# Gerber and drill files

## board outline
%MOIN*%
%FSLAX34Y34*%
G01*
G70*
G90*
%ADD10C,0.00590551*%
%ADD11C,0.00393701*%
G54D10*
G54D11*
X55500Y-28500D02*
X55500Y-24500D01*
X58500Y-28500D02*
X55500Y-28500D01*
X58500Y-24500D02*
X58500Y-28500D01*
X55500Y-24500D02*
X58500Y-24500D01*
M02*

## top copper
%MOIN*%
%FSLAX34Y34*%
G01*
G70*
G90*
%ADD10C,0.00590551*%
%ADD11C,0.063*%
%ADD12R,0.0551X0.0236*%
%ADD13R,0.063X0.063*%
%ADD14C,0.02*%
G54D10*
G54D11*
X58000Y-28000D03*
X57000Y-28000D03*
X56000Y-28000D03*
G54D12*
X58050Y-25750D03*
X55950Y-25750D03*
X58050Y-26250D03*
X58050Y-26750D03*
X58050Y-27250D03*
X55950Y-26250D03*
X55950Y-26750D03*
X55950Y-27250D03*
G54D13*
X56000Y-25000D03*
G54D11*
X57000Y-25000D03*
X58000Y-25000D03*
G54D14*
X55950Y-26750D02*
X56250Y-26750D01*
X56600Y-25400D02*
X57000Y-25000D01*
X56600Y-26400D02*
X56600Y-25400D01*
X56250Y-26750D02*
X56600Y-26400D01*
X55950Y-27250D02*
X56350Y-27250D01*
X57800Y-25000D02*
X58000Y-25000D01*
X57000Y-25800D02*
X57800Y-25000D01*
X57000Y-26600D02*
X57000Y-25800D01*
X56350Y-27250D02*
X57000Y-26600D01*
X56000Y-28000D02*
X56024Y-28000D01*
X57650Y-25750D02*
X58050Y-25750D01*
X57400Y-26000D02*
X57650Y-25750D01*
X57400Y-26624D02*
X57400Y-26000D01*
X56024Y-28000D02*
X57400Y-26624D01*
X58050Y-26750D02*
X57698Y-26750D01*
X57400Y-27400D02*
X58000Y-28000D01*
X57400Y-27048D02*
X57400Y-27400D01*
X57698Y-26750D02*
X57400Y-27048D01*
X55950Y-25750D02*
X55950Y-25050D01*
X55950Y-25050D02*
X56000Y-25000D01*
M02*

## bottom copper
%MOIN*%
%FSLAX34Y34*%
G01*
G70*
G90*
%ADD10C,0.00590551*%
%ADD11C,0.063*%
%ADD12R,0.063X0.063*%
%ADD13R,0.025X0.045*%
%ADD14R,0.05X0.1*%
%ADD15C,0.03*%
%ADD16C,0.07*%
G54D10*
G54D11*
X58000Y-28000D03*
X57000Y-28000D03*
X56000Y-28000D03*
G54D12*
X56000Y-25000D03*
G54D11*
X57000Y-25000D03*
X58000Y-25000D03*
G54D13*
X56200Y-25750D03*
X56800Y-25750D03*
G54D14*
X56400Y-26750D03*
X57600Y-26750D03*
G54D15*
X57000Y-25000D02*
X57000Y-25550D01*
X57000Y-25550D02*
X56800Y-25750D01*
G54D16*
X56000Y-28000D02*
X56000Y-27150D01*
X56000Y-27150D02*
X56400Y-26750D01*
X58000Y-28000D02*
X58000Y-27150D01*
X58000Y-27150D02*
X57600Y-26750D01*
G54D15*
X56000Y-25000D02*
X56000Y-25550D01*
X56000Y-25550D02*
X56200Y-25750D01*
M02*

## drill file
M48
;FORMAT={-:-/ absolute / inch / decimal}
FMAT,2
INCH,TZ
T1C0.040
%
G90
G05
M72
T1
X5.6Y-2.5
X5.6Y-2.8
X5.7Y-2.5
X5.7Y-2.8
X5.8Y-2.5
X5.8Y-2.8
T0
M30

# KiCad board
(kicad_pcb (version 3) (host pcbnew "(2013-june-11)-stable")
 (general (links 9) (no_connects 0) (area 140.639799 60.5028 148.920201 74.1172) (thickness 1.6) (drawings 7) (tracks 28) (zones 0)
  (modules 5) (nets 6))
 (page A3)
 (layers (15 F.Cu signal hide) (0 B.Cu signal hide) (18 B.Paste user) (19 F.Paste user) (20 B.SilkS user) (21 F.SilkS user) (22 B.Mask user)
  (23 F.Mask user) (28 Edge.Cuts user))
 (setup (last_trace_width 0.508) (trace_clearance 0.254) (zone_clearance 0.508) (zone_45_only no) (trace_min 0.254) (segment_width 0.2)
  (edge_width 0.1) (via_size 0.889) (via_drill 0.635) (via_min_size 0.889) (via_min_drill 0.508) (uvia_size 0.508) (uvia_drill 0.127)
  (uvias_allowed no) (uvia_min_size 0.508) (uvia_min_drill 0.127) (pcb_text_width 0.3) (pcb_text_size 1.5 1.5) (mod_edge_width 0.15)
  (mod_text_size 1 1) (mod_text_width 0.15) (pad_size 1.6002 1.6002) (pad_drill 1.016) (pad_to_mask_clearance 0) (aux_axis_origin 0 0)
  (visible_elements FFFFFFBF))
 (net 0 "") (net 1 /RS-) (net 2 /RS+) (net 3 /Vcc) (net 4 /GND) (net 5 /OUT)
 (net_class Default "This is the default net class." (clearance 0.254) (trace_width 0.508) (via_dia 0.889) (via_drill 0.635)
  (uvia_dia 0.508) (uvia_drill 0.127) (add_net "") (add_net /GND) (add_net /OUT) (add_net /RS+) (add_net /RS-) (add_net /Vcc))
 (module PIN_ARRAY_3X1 (layer F.Cu) (at 144.78 71.12 180)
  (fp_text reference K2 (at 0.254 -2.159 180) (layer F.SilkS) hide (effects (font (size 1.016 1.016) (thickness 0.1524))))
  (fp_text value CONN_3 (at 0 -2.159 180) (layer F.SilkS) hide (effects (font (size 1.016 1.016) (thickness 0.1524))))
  (pad 1 thru_hole circle (at -2.54 0 180) (size 1.6002 1.6002) (drill 1.016) (layers *.Cu *.Mask F.SilkS) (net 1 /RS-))
  (pad 2 thru_hole circle (at 0 0 180) (size 1.6002 1.6002) (drill 1.016) (layers *.Cu *.Mask F.SilkS))
  (pad 3 thru_hole circle (at 2.54 0 180) (size 1.6002 1.6002) (drill 1.016) (layers *.Cu *.Mask F.SilkS) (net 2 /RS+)))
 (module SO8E (layer F.Cu) (at 144.78 67.31 270)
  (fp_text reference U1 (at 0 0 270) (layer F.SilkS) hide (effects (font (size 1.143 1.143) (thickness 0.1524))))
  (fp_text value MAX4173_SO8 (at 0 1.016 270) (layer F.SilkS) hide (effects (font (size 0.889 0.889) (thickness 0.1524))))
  (pad 8 smd rect (at -1.905 -2.667 270) (size 0.59944 1.39954) (layers F.Cu F.Paste F.Mask) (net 2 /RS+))
  (pad 1 smd rect (at -1.905 2.667 270) (size 0.59944 1.39954) (layers F.Cu F.Paste F.Mask) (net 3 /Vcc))
  (pad 7 smd rect (at -0.635 -2.667 270) (size 0.59944 1.39954) (layers F.Cu F.Paste F.Mask))
  (pad 6 smd rect (at 0.635 -2.667 270) (size 0.59944 1.39954) (layers F.Cu F.Paste F.Mask) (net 1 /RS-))
  (pad 5 smd rect (at 1.905 -2.667 270) (size 0.59944 1.39954) (layers F.Cu F.Paste F.Mask))
  (pad 2 smd rect (at -0.635 2.667 270) (size 0.59944 1.39954) (layers F.Cu F.Paste F.Mask))
  (pad 3 smd rect (at 0.635 2.667 270) (size 0.59944 1.39954) (layers F.Cu F.Paste F.Mask) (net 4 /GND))
  (pad 4 smd rect (at 1.905 2.667 270) (size 0.59944 1.39954) (layers F.Cu F.Paste F.Mask) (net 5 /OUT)))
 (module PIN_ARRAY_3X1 (layer F.Cu) (at 144.78 63.5)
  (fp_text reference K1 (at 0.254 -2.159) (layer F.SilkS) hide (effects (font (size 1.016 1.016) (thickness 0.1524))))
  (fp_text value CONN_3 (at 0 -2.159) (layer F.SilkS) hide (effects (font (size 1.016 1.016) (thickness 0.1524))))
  (pad 1 thru_hole rect (at -2.54 0) (size 1.6002 1.6002) (drill 1.016) (layers *.Cu *.Mask F.SilkS) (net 3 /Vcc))
  (pad 2 thru_hole circle (at 0 0) (size 1.6002 1.6002) (drill 1.016) (layers *.Cu *.Mask F.SilkS) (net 4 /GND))
  (pad 3 thru_hole circle (at 2.54 0) (size 1.6002 1.6002) (drill 1.016) (layers *.Cu *.Mask F.SilkS) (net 5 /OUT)))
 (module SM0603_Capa (layer B.Cu) (at 143.51 65.405)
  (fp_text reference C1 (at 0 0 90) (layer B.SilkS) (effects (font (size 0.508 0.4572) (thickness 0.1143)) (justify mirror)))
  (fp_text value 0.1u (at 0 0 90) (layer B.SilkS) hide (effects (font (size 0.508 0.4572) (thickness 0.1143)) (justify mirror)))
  (pad 1 smd rect (at -0.762 0) (size 0.635 1.143) (layers B.Cu B.Paste B.Mask) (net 3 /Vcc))
  (pad 2 smd rect (at 0.762 0) (size 0.635 1.143) (layers B.Cu B.Paste B.Mask) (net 4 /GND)))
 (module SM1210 (layer B.Cu) (at 144.78 67.945)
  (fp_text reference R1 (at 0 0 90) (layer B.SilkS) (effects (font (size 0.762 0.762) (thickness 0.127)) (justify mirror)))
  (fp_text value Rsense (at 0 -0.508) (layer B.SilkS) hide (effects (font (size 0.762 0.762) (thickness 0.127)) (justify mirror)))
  (pad 1 smd rect (at -1.524 0) (size 1.27 2.54) (layers B.Cu B.Paste B.Mask) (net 2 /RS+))
  (pad 2 smd rect (at 1.524 0) (size 1.27 2.54) (layers B.Cu B.Paste B.Mask) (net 1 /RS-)))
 (gr_line (start 140.97 72.39) (end 140.97 62.23) (angle 90) (layer Edge.Cuts) (width 0.1))
 (gr_line (start 148.59 72.39) (end 140.97 72.39) (angle 90) (layer Edge.Cuts) (width 0.1))
 (gr_line (start 148.59 62.23) (end 148.59 72.39) (angle 90) (layer Edge.Cuts) (width 0.1))
 (gr_line (start 140.97 62.23) (end 148.59 62.23) (angle 90) (layer Edge.Cuts) (width 0.1))
 (segment (start 144.78 63.5) (end 144.78 64.897) (width 0.762) (layer B.Cu) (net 4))
 (segment (start 144.78 64.897) (end 144.272 65.405) (width 0.762) (layer B.Cu) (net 4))
 (segment (start 142.113 67.945) (end 142.875 67.945) (width 0.508) (layer F.Cu) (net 4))
 (segment (start 143.764 64.516) (end 144.78 63.5) (width 0.508) (layer F.Cu) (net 4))
 (segment (start 143.764 67.056) (end 143.764 64.516) (width 0.508) (layer F.Cu) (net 4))
 (segment (start 142.875 67.945) (end 143.764 67.056) (width 0.508) (layer F.Cu) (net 4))
 (segment (start 142.113 69.215) (end 143.129 69.215) (width 0.508) (layer F.Cu) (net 5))
 (segment (start 146.812 63.5) (end 147.32 63.5) (width 0.508) (layer F.Cu) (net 5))
 (segment (start 144.78 65.532) (end 146.812 63.5) (width 0.508) (layer F.Cu) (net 5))
 (segment (start 144.78 67.564) (end 144.78 65.532) (width 0.508) (layer F.Cu) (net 5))
 (segment (start 143.129 69.215) (end 144.78 67.564) (width 0.508) (layer F.Cu) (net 5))
 (segment (start 142.24 71.12) (end 142.301634 71.12) (width 0.508) (layer F.Cu) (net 2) (status C00000))
 (segment (start 146.431 65.405) (end 147.447 65.405) (width 0.508) (layer F.Cu) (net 2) (status 800000))
 (segment (start 145.796 66.04) (end 146.431 65.405) (width 0.508) (layer F.Cu) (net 2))
 (segment (start 145.796 67.625634) (end 145.796 66.04) (width 0.508) (layer F.Cu) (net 2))
 (segment (start 142.301634 71.12) (end 145.796 67.625634) (width 0.508) (layer F.Cu) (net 2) (status 400000))
 (segment (start 142.24 71.12) (end 142.24 68.961) (width 1.778) (layer B.Cu) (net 2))
 (segment (start 142.24 68.961) (end 143.256 67.945) (width 1.778) (layer B.Cu) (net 2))
 (segment (start 147.447 67.945) (end 146.554268 67.945) (width 0.508) (layer F.Cu) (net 1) (status 400000))
 (segment (start 145.796 69.596) (end 147.32 71.12) (width 0.508) (layer F.Cu) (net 1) (status 800000))
 (segment (start 145.796 68.703268) (end 145.796 69.596) (width 0.508) (layer F.Cu) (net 1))
 (segment (start 146.554268 67.945) (end 145.796 68.703268) (width 0.508) (layer F.Cu) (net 1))
 (segment (start 147.32 71.12) (end 147.32 68.961) (width 1.778) (layer B.Cu) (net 1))
 (segment (start 147.32 68.961) (end 146.304 67.945) (width 1.778) (layer B.Cu) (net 1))
 (segment (start 142.24 63.5) (end 142.24 64.897) (width 0.762) (layer B.Cu) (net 3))
 (segment (start 142.24 64.897) (end 142.748 65.405) (width 0.762) (layer B.Cu) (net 3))
 (segment (start 142.113 65.405) (end 142.113 63.627) (width 0.508) (layer F.Cu) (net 3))
 (segment (start 142.113 63.627) (end 142.24 63.5) (width 0.508) (layer F.Cu) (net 3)))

